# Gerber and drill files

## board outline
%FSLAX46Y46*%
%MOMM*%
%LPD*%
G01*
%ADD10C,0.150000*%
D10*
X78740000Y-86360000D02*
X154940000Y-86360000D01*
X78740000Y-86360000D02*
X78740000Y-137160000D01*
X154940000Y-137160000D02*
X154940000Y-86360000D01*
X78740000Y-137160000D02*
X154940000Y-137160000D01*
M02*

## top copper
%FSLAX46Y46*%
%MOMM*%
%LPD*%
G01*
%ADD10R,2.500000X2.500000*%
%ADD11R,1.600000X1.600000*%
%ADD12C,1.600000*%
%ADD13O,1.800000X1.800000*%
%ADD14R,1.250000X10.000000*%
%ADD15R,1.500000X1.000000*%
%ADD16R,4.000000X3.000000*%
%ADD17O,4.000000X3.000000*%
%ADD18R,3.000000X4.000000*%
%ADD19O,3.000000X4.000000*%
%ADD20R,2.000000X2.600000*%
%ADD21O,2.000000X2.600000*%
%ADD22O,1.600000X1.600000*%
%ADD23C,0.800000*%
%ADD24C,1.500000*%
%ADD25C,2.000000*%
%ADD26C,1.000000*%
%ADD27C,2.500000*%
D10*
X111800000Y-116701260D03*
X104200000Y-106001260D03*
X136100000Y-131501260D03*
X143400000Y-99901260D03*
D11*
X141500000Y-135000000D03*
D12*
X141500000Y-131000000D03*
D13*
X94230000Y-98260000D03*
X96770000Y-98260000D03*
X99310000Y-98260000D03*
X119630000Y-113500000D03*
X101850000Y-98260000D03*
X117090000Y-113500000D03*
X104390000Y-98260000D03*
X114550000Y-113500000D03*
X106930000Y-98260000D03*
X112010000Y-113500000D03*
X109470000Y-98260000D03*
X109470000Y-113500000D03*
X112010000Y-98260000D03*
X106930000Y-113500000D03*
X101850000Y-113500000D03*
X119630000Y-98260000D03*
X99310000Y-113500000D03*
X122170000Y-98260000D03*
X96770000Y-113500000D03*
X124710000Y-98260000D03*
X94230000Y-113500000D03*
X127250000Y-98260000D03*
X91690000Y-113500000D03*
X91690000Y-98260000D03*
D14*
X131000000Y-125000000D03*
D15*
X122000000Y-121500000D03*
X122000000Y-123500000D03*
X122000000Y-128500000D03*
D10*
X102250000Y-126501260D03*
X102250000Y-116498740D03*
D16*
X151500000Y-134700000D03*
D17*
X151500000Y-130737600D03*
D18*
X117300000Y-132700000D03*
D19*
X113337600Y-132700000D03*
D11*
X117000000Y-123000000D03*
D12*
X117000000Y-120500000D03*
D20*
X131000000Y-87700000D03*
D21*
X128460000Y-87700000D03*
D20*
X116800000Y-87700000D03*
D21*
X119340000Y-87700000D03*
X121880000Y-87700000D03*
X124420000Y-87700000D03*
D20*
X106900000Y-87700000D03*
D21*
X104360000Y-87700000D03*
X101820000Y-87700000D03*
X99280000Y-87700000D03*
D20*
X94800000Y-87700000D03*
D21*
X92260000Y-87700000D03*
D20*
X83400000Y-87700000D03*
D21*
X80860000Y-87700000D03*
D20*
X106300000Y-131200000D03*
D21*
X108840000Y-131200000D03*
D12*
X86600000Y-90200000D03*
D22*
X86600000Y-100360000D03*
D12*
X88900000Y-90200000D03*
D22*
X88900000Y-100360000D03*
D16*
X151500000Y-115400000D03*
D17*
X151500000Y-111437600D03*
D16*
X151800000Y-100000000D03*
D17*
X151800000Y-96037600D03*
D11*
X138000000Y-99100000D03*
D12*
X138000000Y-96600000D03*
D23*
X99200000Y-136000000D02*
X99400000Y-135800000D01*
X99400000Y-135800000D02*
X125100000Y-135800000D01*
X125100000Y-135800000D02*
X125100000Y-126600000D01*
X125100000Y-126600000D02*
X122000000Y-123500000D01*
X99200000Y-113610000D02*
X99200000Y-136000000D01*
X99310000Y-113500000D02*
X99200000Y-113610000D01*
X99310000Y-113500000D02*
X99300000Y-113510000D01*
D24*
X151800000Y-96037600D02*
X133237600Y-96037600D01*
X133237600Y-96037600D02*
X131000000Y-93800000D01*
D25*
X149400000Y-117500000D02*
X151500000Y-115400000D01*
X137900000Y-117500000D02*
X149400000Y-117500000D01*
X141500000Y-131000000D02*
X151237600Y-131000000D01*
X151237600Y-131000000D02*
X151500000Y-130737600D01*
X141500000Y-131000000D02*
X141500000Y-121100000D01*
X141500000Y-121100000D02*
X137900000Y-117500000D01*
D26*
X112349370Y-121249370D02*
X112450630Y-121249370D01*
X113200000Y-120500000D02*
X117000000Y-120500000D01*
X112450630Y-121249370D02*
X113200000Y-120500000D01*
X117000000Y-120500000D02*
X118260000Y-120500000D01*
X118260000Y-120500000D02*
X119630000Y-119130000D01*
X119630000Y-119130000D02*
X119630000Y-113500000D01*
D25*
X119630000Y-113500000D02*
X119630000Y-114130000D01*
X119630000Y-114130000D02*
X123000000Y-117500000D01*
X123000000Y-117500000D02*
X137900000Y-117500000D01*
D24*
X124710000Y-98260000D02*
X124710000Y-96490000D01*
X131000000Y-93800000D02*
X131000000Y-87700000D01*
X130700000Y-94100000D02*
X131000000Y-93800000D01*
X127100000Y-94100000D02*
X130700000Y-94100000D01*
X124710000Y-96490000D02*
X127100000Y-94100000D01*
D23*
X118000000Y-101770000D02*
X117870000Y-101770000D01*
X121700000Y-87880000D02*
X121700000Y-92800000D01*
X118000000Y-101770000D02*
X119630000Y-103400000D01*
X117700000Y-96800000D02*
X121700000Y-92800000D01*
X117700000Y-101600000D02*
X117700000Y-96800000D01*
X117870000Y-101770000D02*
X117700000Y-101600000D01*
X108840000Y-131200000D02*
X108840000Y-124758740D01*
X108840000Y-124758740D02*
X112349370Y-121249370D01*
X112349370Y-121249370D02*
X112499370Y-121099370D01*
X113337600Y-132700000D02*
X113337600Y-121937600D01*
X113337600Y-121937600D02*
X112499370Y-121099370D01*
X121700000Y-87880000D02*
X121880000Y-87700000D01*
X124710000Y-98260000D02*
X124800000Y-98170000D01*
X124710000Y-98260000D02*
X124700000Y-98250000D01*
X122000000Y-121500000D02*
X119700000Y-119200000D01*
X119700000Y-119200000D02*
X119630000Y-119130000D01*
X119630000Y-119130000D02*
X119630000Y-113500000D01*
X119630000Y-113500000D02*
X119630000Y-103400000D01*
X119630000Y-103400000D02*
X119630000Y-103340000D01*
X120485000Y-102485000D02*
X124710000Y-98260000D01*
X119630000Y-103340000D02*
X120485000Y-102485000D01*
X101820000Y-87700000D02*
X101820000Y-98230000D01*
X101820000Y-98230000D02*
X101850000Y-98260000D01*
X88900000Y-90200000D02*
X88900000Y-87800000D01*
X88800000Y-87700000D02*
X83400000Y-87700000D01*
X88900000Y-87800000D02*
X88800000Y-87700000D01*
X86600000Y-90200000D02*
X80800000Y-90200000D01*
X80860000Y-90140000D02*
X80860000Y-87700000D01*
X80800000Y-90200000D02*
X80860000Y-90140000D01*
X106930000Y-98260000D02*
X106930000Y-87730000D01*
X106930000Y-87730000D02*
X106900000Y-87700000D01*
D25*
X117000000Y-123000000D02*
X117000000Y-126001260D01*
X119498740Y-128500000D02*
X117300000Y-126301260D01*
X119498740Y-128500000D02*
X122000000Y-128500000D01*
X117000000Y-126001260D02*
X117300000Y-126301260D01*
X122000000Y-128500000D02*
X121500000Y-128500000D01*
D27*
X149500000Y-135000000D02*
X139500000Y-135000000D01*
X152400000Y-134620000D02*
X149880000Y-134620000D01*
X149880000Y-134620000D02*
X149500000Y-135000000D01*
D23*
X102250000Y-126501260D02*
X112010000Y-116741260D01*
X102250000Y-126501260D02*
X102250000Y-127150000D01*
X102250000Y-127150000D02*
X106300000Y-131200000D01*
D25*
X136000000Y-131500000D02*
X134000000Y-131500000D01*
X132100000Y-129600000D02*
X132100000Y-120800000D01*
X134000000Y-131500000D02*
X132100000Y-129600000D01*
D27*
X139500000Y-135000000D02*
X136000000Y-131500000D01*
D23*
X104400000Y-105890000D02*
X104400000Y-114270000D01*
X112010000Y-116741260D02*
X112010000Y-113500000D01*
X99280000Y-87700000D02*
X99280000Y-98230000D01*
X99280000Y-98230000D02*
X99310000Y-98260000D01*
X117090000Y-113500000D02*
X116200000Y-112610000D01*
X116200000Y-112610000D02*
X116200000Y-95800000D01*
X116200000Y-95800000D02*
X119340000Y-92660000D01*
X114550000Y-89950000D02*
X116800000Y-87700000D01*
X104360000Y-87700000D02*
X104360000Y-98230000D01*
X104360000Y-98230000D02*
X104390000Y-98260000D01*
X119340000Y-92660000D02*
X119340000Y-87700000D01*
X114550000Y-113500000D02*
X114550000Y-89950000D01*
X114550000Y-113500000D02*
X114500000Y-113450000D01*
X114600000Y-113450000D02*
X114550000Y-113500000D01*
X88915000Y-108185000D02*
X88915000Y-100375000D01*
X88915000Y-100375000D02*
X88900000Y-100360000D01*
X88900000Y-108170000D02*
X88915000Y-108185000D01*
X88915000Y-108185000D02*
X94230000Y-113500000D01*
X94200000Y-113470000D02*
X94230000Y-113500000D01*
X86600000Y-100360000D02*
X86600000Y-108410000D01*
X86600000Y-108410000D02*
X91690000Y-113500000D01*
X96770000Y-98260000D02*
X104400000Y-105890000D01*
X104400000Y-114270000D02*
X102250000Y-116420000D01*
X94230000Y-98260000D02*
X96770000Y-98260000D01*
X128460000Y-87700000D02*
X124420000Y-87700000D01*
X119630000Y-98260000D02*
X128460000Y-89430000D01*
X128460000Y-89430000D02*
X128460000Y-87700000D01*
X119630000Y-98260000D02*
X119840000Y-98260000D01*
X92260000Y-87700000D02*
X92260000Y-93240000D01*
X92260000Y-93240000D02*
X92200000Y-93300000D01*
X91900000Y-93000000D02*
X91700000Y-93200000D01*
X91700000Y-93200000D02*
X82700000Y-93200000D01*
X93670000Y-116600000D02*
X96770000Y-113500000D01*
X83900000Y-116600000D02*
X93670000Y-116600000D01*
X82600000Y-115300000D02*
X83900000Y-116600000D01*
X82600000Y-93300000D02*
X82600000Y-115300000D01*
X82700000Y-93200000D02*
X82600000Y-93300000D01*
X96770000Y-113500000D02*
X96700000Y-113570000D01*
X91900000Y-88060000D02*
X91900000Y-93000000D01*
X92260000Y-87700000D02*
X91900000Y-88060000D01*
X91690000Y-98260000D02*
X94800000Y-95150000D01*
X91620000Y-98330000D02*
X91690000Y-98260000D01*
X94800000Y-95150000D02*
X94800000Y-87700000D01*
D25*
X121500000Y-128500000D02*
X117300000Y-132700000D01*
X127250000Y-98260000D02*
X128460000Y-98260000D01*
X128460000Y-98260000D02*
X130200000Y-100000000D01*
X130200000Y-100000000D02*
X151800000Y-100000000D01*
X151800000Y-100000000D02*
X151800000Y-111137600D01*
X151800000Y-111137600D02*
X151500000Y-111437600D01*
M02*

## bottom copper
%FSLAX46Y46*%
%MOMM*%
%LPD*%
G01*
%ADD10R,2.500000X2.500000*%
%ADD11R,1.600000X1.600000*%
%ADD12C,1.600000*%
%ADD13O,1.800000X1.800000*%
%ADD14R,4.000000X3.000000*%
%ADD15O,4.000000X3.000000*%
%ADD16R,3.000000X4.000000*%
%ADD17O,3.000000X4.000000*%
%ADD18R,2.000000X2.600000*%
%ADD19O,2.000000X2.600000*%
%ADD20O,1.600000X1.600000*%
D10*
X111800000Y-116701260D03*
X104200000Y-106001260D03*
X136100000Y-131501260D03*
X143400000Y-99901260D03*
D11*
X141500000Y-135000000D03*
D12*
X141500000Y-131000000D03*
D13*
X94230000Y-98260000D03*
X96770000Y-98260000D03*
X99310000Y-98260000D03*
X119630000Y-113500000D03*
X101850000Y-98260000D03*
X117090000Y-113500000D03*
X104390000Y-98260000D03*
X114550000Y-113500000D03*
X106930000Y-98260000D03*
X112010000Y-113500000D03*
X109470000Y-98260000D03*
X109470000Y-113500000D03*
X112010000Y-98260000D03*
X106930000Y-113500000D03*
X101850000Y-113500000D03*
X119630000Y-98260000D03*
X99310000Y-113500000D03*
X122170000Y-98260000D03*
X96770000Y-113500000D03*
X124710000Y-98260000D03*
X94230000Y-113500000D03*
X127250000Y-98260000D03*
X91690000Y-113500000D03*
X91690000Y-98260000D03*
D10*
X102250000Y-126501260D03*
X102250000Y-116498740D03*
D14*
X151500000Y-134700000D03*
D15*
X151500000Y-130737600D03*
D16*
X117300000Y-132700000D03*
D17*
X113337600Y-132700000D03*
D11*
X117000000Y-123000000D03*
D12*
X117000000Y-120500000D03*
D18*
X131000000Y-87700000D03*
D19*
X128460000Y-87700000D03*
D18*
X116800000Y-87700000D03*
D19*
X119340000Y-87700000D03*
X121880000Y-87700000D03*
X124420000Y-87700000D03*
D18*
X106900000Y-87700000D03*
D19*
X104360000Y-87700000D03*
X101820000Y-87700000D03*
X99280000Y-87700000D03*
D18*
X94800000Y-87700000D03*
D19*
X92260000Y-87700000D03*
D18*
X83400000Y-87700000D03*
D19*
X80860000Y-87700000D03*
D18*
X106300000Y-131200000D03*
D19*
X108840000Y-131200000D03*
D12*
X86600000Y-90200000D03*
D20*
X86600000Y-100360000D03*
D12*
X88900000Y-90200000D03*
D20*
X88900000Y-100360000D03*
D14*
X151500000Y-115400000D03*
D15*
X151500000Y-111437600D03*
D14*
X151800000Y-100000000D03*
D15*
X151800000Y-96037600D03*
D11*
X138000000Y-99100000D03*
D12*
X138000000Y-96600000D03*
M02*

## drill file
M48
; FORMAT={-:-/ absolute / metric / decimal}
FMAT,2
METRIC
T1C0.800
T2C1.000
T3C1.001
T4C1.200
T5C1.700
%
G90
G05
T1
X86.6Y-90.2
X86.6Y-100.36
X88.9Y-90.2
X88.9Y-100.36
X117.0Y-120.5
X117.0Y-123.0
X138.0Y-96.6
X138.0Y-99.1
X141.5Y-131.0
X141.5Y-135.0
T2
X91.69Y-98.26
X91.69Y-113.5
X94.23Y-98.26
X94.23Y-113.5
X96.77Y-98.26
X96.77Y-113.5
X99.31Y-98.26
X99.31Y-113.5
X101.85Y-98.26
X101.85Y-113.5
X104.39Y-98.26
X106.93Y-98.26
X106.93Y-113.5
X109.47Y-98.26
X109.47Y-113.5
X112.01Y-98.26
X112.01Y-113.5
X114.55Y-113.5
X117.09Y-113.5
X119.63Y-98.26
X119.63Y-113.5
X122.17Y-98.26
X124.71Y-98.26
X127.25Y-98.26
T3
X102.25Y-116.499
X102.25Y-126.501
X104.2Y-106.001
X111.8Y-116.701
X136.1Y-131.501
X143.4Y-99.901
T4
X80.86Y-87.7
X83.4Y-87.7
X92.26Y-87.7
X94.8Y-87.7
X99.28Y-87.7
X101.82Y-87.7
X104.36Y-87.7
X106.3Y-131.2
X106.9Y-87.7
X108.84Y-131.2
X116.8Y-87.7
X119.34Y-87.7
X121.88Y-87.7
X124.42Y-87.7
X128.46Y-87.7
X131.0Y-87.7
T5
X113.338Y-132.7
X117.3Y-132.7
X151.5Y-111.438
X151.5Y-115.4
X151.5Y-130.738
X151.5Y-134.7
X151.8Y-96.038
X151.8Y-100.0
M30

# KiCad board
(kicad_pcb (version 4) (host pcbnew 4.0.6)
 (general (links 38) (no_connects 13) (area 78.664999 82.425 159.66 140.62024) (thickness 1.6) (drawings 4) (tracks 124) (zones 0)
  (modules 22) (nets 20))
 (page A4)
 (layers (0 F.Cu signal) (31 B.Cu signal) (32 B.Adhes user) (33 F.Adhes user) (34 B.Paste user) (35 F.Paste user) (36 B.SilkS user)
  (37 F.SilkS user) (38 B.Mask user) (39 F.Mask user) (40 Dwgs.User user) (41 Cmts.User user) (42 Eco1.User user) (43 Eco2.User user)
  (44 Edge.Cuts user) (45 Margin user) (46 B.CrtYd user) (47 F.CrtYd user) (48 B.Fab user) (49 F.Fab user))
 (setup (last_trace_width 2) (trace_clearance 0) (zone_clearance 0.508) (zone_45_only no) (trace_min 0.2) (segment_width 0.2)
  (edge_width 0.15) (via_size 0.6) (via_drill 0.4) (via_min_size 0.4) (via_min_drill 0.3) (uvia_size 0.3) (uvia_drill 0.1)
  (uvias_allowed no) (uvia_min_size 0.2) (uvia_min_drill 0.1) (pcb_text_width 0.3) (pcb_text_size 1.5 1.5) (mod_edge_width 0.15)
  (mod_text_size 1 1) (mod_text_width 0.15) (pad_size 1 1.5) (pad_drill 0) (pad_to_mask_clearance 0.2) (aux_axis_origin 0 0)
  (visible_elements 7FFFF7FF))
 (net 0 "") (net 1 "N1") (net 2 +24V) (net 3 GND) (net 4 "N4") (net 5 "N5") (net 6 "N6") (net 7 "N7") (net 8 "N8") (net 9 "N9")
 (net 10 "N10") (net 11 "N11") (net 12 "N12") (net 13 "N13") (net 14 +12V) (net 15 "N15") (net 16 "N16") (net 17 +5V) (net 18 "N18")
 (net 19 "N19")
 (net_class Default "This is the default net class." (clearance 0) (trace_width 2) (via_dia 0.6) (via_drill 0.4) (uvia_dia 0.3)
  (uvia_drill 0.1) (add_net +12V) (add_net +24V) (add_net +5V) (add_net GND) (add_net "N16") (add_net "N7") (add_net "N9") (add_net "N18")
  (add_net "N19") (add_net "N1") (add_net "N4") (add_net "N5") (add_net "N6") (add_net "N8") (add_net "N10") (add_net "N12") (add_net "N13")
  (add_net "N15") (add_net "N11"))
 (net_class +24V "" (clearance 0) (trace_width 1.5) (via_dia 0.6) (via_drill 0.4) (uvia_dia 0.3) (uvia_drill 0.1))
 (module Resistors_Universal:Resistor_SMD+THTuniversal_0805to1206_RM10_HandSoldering (layer F.Cu) (at 111.8 111.7 90)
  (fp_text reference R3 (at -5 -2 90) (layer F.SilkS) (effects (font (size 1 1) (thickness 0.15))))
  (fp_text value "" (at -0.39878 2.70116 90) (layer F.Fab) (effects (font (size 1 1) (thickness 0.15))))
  (pad 1 thru_hole rect (at -5.00126 0 270) (size 2.5 2.5) (drill 1.00076) (layers *.Cu *.Mask) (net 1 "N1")))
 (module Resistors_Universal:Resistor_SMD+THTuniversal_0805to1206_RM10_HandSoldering (layer F.Cu) (at 104.2 101 90)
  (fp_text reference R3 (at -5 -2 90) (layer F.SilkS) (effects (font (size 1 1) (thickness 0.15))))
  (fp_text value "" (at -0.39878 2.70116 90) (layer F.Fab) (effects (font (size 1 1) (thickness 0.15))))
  (pad 1 thru_hole rect (at -5.00126 0 270) (size 2.5 2.5) (drill 1.00076) (layers *.Cu *.Mask) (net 1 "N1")))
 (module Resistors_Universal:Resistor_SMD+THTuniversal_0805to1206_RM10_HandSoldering (layer F.Cu) (at 136.1 126.5 90)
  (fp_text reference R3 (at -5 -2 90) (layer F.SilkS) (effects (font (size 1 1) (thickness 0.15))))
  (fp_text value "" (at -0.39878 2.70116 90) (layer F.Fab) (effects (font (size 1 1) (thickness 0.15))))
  (pad 1 thru_hole rect (at -5.00126 0 270) (size 2.5 2.5) (drill 1.00076) (layers *.Cu *.Mask) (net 1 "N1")))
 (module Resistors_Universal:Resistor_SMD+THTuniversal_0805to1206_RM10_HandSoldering (layer F.Cu) (at 143.4 94.9 90)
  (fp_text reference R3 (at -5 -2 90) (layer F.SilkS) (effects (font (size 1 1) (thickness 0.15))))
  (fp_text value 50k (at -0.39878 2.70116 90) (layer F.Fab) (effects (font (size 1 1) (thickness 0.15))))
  (pad 1 thru_hole rect (at -5.00126 0 270) (size 2.5 2.5) (drill 1.00076) (layers *.Cu *.Mask) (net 1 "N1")))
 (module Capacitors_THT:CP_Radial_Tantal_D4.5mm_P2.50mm (layer B.Cu) (at 141.5 135 90)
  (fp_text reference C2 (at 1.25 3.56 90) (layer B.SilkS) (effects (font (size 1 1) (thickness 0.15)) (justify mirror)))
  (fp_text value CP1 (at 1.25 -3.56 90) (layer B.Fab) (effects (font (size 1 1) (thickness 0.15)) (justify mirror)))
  (pad 1 thru_hole rect (at 0 0 90) (size 1.6 1.6) (drill 0.8) (layers *.Cu *.Mask) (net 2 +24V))
  (pad 2 thru_hole circle (at 4 0 90) (size 1.6 1.6) (drill 0.8) (layers *.Cu *.Mask) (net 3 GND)))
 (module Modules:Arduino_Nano (layer B.Cu) (at 127.25 113.5 90)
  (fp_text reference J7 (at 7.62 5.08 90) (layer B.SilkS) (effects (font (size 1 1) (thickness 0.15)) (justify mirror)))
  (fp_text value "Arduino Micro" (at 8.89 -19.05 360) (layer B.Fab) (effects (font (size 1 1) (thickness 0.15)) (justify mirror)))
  (pad 3.3V thru_hole oval (at 15.24 -33.02 90) (size 1.8 1.8) (drill 1) (layers *.Cu *.Mask) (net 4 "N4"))
  (pad AREF thru_hole oval (at 15.24 -30.48 90) (size 1.8 1.8) (drill 1) (layers *.Cu *.Mask) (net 4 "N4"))
  (pad A0 thru_hole oval (at 15.24 -27.94 90) (size 1.8 1.8) (drill 1) (layers *.Cu *.Mask) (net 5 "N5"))
  (pad GND thru_hole oval (at 0 -7.62 90) (size 1.8 1.8) (drill 1) (layers *.Cu *.Mask) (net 3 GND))
  (pad A1 thru_hole oval (at 15.24 -25.4 90) (size 1.8 1.8) (drill 1) (layers *.Cu *.Mask) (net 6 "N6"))
  (pad SDA thru_hole oval (at 0 -10.16 90) (size 1.8 1.8) (drill 1) (layers *.Cu *.Mask) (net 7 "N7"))
  (pad A2 thru_hole oval (at 15.24 -22.86 90) (size 1.8 1.8) (drill 1) (layers *.Cu *.Mask) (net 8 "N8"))
  (pad SCL thru_hole oval (at 0 -12.7 90) (size 1.8 1.8) (drill 1) (layers *.Cu *.Mask) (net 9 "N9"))
  (pad A3 thru_hole oval (at 15.24 -20.32 90) (size 1.8 1.8) (drill 1) (layers *.Cu *.Mask) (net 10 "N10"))
  (pad D4 thru_hole oval (at 0 -15.24 90) (size 1.8 1.8) (drill 1) (layers *.Cu *.Mask) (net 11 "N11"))
  (pad A4 thru_hole oval (at 15.24 -17.78 90) (size 1.8 1.8) (drill 1) (layers *.Cu *.Mask) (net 1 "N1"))
  (pad D5 thru_hole oval (at 0 -17.78 90) (size 1.8 1.8) (drill 1) (layers *.Cu *.Mask))
  (pad A5 thru_hole oval (at 15.24 -15.24 90) (size 1.8 1.8) (drill 1) (layers *.Cu *.Mask) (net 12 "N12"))
  (pad D6 thru_hole oval (at 0 -20.32 90) (size 1.8 1.8) (drill 1) (layers *.Cu *.Mask))
  (pad D8 thru_hole oval (at 0 -25.4 90) (size 1.8 1.8) (drill 1) (layers *.Cu *.Mask))
  (pad 5v thru_hole oval (at 15.24 -7.62 90) (size 1.8 1.8) (drill 1) (layers *.Cu *.Mask))
  (pad D9 thru_hole oval (at 0 -27.94 90) (size 1.8 1.8) (drill 1) (layers *.Cu *.Mask))
  (pad RS thru_hole oval (at 15.24 -5.08 90) (size 1.8 1.8) (drill 1) (layers *.Cu *.Mask))
  (pad D10 thru_hole oval (at 0 -30.48 90) (size 1.8 1.8) (drill 1) (layers *.Cu *.Mask))
  (pad GND thru_hole oval (at 15.24 -2.54 90) (size 1.8 1.8) (drill 1) (layers *.Cu *.Mask) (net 3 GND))
  (pad D11 thru_hole oval (at 0 -33.02 90) (size 1.8 1.8) (drill 1) (layers *.Cu *.Mask) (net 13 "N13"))
  (pad Vin thru_hole oval (at 15.24 0 90) (size 1.8 1.8) (drill 1) (layers *.Cu *.Mask) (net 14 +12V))
  (pad D12 thru_hole oval (at 0 -35.56 90) (size 1.8 1.8) (drill 1) (layers *.Cu *.Mask) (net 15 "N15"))
  (pad D13 thru_hole oval (at 15.24 -35.56 90) (size 1.8 1.8) (drill 1) (layers *.Cu *.Mask)))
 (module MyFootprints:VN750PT (layer F.Cu) (at 128 125 270)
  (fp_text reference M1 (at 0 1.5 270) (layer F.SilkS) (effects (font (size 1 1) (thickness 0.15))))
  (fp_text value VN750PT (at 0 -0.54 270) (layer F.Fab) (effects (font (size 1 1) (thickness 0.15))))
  (pad Vcc smd rect (at 0 -3 270) (size 10 1.25) (layers F.Cu F.Paste F.Mask))
  (pad GND smd rect (at -3.5 6 270) (size 1 1.5) (layers F.Cu F.Paste F.Mask))
  (pad Inpu smd rect (at -1.5 6 270) (size 1 1.5) (layers F.Cu F.Paste F.Mask))
  (pad Vout smd rect (at 3.5 6 270) (size 1 1.5) (layers F.Cu F.Paste F.Mask) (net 2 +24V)))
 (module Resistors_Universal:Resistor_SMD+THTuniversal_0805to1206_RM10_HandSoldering (layer F.Cu) (at 102.25 121.5 90)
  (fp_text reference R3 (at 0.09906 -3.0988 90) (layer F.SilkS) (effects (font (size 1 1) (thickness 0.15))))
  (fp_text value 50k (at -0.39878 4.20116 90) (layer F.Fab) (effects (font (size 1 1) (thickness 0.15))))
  (pad 1 thru_hole rect (at -5.00126 0 270) (size 2.5 2.5) (drill 1.00076) (layers *.Cu *.Mask) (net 1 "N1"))
  (pad 2 thru_hole rect (at 5.00126 0 270) (size 2.5 2.5) (drill 1.00076) (layers *.Cu *.Mask) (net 4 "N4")))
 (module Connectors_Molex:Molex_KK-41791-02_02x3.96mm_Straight (layer F.Cu) (at 151.5 134.7 90)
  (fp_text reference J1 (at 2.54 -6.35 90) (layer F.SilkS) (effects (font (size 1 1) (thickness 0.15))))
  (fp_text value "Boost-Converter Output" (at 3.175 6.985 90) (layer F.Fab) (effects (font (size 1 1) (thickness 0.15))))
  (pad 1 thru_hole rect (at 0 0 90) (size 3 4) (drill 1.7) (layers *.Cu *.Mask) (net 2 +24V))
  (pad 2 thru_hole oval (at 3.9624 0 90) (size 3 4) (drill 1.7) (layers *.Cu *.Mask) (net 3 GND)))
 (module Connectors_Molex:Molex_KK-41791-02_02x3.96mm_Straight (layer B.Cu) (at 117.3 132.7 180)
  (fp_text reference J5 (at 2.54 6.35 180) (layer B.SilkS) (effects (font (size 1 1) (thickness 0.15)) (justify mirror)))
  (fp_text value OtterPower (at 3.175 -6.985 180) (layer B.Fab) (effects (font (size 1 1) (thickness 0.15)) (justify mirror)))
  (pad 1 thru_hole rect (at 0 0 180) (size 3 4) (drill 1.7) (layers *.Cu *.Mask) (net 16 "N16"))
  (pad 2 thru_hole oval (at 3.9624 0 180) (size 3 4) (drill 1.7) (layers *.Cu *.Mask) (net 3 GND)))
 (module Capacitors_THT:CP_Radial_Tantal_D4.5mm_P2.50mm (layer B.Cu) (at 117 123 90)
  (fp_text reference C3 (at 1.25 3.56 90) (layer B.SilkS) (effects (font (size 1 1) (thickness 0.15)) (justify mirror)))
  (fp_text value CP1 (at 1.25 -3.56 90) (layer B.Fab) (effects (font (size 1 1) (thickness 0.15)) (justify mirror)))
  (pad + thru_hole rect (at 0 0 90) (size 1.6 1.6) (drill 0.8) (layers *.Cu *.Mask) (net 2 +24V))
  (pad 2 thru_hole circle (at 2.5 0 90) (size 1.6 1.6) (drill 0.8) (layers *.Cu *.Mask) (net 3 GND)))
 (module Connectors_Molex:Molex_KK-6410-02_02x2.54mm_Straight (layer F.Cu) (at 131 87.7 180)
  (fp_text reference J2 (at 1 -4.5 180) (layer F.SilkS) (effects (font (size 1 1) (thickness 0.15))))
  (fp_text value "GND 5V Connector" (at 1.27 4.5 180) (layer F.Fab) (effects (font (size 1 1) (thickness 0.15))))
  (pad 1 thru_hole rect (at 0 0 180) (size 2 2.6) (drill 1.2) (layers *.Cu *.Mask) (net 3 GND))
  (pad 2 thru_hole oval (at 2.54 0 180) (size 2 2.6) (drill 1.2) (layers *.Cu *.Mask) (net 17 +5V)))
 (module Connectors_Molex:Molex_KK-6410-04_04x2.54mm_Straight (layer B.Cu) (at 116.8 87.7)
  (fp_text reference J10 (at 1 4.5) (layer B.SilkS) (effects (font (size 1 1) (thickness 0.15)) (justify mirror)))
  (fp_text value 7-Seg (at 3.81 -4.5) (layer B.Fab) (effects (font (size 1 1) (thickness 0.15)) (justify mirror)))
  (pad 1 thru_hole rect (at 0 0) (size 2 2.6) (drill 1.2) (layers *.Cu *.Mask) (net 7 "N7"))
  (pad 2 thru_hole oval (at 2.54 0) (size 2 2.6) (drill 1.2) (layers *.Cu *.Mask) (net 9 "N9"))
  (pad 3 thru_hole oval (at 5.08 0) (size 2 2.6) (drill 1.2) (layers *.Cu *.Mask) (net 3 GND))
  (pad 4 thru_hole oval (at 7.62 0) (size 2 2.6) (drill 1.2) (layers *.Cu *.Mask) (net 17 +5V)))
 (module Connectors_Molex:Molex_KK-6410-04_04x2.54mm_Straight (layer F.Cu) (at 106.9 87.7 180)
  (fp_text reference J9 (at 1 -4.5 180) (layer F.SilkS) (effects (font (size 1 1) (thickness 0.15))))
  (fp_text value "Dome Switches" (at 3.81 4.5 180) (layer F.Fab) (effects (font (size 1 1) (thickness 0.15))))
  (pad 1 thru_hole rect (at 0 0 180) (size 2 2.6) (drill 1.2) (layers *.Cu *.Mask) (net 10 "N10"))
  (pad 2 thru_hole oval (at 2.54 0 180) (size 2 2.6) (drill 1.2) (layers *.Cu *.Mask) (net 8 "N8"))
  (pad 3 thru_hole oval (at 5.08 0 180) (size 2 2.6) (drill 1.2) (layers *.Cu *.Mask) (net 6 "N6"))
  (pad 4 thru_hole oval (at 7.62 0 180) (size 2 2.6) (drill 1.2) (layers *.Cu *.Mask) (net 5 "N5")))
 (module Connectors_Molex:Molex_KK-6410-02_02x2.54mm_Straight (layer F.Cu) (at 94.8 87.7 180)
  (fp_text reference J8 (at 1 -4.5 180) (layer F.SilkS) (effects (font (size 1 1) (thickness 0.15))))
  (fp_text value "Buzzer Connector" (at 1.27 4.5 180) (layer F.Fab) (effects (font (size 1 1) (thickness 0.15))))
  (pad 1 thru_hole rect (at 0 0 180) (size 2 2.6) (drill 1.2) (layers *.Cu *.Mask) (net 12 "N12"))
  (pad 2 thru_hole oval (at 2.54 0 180) (size 2 2.6) (drill 1.2) (layers *.Cu *.Mask) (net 11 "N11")))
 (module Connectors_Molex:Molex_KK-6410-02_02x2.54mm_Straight (layer F.Cu) (at 83.4 87.7 180)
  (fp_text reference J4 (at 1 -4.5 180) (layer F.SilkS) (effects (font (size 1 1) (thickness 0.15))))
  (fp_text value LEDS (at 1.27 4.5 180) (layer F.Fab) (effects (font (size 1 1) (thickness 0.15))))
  (pad 1 thru_hole rect (at 0 0 180) (size 2 2.6) (drill 1.2) (layers *.Cu *.Mask) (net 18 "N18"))
  (pad 2 thru_hole oval (at 2.54 0 180) (size 2 2.6) (drill 1.2) (layers *.Cu *.Mask) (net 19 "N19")))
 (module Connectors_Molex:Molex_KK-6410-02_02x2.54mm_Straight (layer F.Cu) (at 106.3 131.2)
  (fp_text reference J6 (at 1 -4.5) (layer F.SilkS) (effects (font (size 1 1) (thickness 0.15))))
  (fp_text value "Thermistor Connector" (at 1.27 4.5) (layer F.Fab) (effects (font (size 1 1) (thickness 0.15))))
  (pad 1 thru_hole rect (at 0 0) (size 2 2.6) (drill 1.2) (layers *.Cu *.Mask) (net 1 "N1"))
  (pad 2 thru_hole oval (at 2.54 0) (size 2 2.6) (drill 1.2) (layers *.Cu *.Mask) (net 3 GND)))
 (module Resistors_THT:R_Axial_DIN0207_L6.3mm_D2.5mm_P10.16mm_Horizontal (layer F.Cu) (at 86.6 90.2 270)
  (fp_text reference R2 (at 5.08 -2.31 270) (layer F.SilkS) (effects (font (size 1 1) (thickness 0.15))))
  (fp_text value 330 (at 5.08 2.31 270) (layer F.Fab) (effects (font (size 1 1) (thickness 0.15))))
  (pad 1 thru_hole circle (at 0 0 270) (size 1.6 1.6) (drill 0.8) (layers *.Cu *.Mask) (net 19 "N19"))
  (pad 2 thru_hole oval (at 10.16 0 270) (size 1.6 1.6) (drill 0.8) (layers *.Cu *.Mask) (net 15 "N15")))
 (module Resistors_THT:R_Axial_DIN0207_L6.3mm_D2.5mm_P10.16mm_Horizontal (layer F.Cu) (at 88.9 90.2 270)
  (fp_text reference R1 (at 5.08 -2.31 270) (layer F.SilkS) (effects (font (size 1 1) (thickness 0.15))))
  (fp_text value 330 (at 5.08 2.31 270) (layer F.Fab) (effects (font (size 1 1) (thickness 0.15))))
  (pad 1 thru_hole circle (at 0 0 270) (size 1.6 1.6) (drill 0.8) (layers *.Cu *.Mask) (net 18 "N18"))
  (pad 2 thru_hole oval (at 10.16 0 270) (size 1.6 1.6) (drill 0.8) (layers *.Cu *.Mask) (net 13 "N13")))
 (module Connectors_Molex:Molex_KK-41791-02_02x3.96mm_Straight (layer F.Cu) (at 151.5 115.4 90)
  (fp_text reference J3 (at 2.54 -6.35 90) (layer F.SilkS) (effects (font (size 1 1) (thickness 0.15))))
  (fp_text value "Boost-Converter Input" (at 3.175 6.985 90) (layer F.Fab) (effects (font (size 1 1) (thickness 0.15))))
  (pad 1 thru_hole rect (at 0 0 90) (size 3 4) (drill 1.7) (layers *.Cu *.Mask) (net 3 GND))
  (pad 2 thru_hole oval (at 3.9624 0 90) (size 3 4) (drill 1.7) (layers *.Cu *.Mask) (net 14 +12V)))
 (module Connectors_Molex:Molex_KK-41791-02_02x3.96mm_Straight (layer F.Cu) (at 151.8 100 90)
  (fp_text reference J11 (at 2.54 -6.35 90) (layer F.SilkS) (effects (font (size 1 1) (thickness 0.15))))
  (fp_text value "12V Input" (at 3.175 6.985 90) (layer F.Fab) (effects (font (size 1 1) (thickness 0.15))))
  (pad 1 thru_hole rect (at 0 0 90) (size 3 4) (drill 1.7) (layers *.Cu *.Mask) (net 14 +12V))
  (pad 2 thru_hole oval (at 3.9624 0 90) (size 3 4) (drill 1.7) (layers *.Cu *.Mask) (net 3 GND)))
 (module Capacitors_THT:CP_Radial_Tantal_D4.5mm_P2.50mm (layer F.Cu) (at 138 99.1 90)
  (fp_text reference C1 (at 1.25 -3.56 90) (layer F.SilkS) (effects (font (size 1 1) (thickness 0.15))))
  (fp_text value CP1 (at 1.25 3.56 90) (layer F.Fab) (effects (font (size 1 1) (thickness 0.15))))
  (pad 1 thru_hole rect (at 0 0 90) (size 1.6 1.6) (drill 0.8) (layers *.Cu *.Mask) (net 16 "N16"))
  (pad 2 thru_hole circle (at 2.5 0 90) (size 1.6 1.6) (drill 0.8) (layers *.Cu *.Mask) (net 3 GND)))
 (gr_line (start 78.74 86.36) (end 154.94 86.36) (angle 90) (layer Edge.Cuts) (width 0.15))
 (gr_line (start 78.74 86.36) (end 78.74 137.16) (angle 90) (layer Edge.Cuts) (width 0.15))
 (gr_line (start 154.94 137.16) (end 154.94 86.36) (angle 90) (layer Edge.Cuts) (width 0.15))
 (gr_line (start 78.74 137.16) (end 154.94 137.16) (angle 90) (layer Edge.Cuts) (width 0.15))
 (segment (start 99.2 136) (end 99.4 135.8) (width 0.8) (layer F.Cu) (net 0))
 (segment (start 99.4 135.8) (end 125.1 135.8) (width 0.8) (layer F.Cu) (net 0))
 (segment (start 125.1 135.8) (end 125.1 126.6) (width 0.8) (layer F.Cu) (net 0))
 (segment (start 125.1 126.6) (end 122 123.5) (width 0.8) (layer F.Cu) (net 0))
 (segment (start 99.2 113.61) (end 99.2 136) (width 0.8) (layer F.Cu) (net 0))
 (segment (start 99.31 113.5) (end 99.2 113.61) (width 0.8) (layer F.Cu) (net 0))
 (segment (start 99.31 113.5) (end 99.3 113.51) (width 0.8) (layer F.Cu) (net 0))
 (segment (start 151.8 96.0376) (end 133.2376 96.0376) (width 1.5) (layer F.Cu) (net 3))
 (segment (start 133.2376 96.0376) (end 131 93.8) (width 1.5) (layer F.Cu) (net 3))
 (segment (start 149.4 117.5) (end 151.5 115.4) (width 2) (layer F.Cu) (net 3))
 (segment (start 137.9 117.5) (end 149.4 117.5) (width 2) (layer F.Cu) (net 3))
 (segment (start 141.5 131) (end 151.2376 131) (width 2) (layer F.Cu) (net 3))
 (segment (start 151.2376 131) (end 151.5 130.7376) (width 2) (layer F.Cu) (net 3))
 (segment (start 141.5 131) (end 141.5 121.1) (width 2) (layer F.Cu) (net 3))
 (segment (start 141.5 121.1) (end 137.9 117.5) (width 2) (layer F.Cu) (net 3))
 (segment (start 112.34937 121.24937) (end 112.45063 121.24937) (width 1) (layer F.Cu) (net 3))
 (segment (start 113.2 120.5) (end 117 120.5) (width 1) (layer F.Cu) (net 3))
 (segment (start 112.45063 121.24937) (end 113.2 120.5) (width 1) (layer F.Cu) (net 3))
 (segment (start 117 120.5) (end 118.26 120.5) (width 1) (layer F.Cu) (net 3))
 (segment (start 118.26 120.5) (end 119.63 119.13) (width 1) (layer F.Cu) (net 3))
 (segment (start 119.63 119.13) (end 119.63 113.5) (width 1) (layer F.Cu) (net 3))
 (segment (start 119.63 113.5) (end 119.63 114.13) (width 2) (layer F.Cu) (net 3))
 (segment (start 119.63 114.13) (end 123 117.5) (width 2) (layer F.Cu) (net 3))
 (segment (start 123 117.5) (end 137.9 117.5) (width 2) (layer F.Cu) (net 3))
 (segment (start 124.71 98.26) (end 124.71 96.49) (width 1.5) (layer F.Cu) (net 3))
 (segment (start 131 93.8) (end 131 87.7) (width 1.5) (layer F.Cu) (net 3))
 (segment (start 130.7 94.1) (end 131 93.8) (width 1.5) (layer F.Cu) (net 3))
 (segment (start 127.1 94.1) (end 130.7 94.1) (width 1.5) (layer F.Cu) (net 3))
 (segment (start 124.71 96.49) (end 127.1 94.1) (width 1.5) (layer F.Cu) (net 3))
 (segment (start 118 101.77) (end 117.87 101.77) (width 0.8) (layer F.Cu) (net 3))
 (segment (start 121.7 87.88) (end 121.7 92.8) (width 0.8) (layer F.Cu) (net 3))
 (segment (start 118 101.77) (end 119.63 103.4) (width 0.8) (layer F.Cu) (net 3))
 (segment (start 117.7 96.8) (end 121.7 92.8) (width 0.8) (layer F.Cu) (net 3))
 (segment (start 117.7 101.6) (end 117.7 96.8) (width 0.8) (layer F.Cu) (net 3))
 (segment (start 117.87 101.77) (end 117.7 101.6) (width 0.8) (layer F.Cu) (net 3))
 (segment (start 108.84 131.2) (end 108.84 124.75874) (width 0.8) (layer F.Cu) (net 3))
 (segment (start 108.84 124.75874) (end 112.34937 121.24937) (width 0.8) (layer F.Cu) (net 3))
 (segment (start 112.34937 121.24937) (end 112.49937 121.09937) (width 0.8) (layer F.Cu) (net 3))
 (segment (start 113.3376 132.7) (end 113.3376 121.9376) (width 0.8) (layer F.Cu) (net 3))
 (segment (start 113.3376 121.9376) (end 112.49937 121.09937) (width 0.8) (layer F.Cu) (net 3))
 (segment (start 121.7 87.88) (end 121.88 87.7) (width 0.8) (layer F.Cu) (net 3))
 (segment (start 124.71 98.26) (end 124.8 98.17) (width 0.8) (layer F.Cu) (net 3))
 (segment (start 124.71 98.26) (end 124.7 98.25) (width 0.8) (layer F.Cu) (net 3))
 (segment (start 122 121.5) (end 119.7 119.2) (width 0.8) (layer F.Cu) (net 3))
 (segment (start 119.7 119.2) (end 119.63 119.13) (width 0.8) (layer F.Cu) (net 3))
 (segment (start 119.63 119.13) (end 119.63 113.5) (width 0.8) (layer F.Cu) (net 3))
 (segment (start 119.63 113.5) (end 119.63 103.4) (width 0.8) (layer F.Cu) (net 3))
 (segment (start 119.63 103.4) (end 119.63 103.34) (width 0.8) (layer F.Cu) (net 3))
 (segment (start 120.485 102.485) (end 124.71 98.26) (width 0.8) (layer F.Cu) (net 3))
 (segment (start 119.63 103.34) (end 120.485 102.485) (width 0.8) (layer F.Cu) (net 3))
 (segment (start 101.82 87.7) (end 101.82 98.23) (width 0.8) (layer F.Cu) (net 6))
 (segment (start 101.82 98.23) (end 101.85 98.26) (width 0.8) (layer F.Cu) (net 6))
 (segment (start 88.9 90.2) (end 88.9 87.8) (width 0.8) (layer F.Cu) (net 18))
 (segment (start 88.8 87.7) (end 83.4 87.7) (width 0.8) (layer F.Cu) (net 18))
 (segment (start 88.9 87.8) (end 88.8 87.7) (width 0.8) (layer F.Cu) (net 18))
 (segment (start 86.6 90.2) (end 80.8 90.2) (width 0.8) (layer F.Cu) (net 19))
 (segment (start 80.86 90.14) (end 80.86 87.7) (width 0.8) (layer F.Cu) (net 19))
 (segment (start 80.8 90.2) (end 80.86 90.14) (width 0.8) (layer F.Cu) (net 19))
 (segment (start 106.93 98.26) (end 106.93 87.73) (width 0.8) (layer F.Cu) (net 10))
 (segment (start 106.93 87.73) (end 106.9 87.7) (width 0.8) (layer F.Cu) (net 10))
 (segment (start 117 123) (end 117 126.00126) (width 2) (layer F.Cu) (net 2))
 (segment (start 119.49874 128.5) (end 117.3 126.30126) (width 2) (layer F.Cu) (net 2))
 (segment (start 119.49874 128.5) (end 122 128.5) (width 2) (layer F.Cu) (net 2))
 (segment (start 117 126.00126) (end 117.3 126.30126) (width 2) (layer F.Cu) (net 2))
 (segment (start 122 128.5) (end 121.5 128.5) (width 2) (layer F.Cu) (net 2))
 (segment (start 149.5 135) (end 139.5 135) (width 2.5) (layer F.Cu) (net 2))
 (segment (start 152.4 134.62) (end 149.88 134.62) (width 2.5) (layer F.Cu) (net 2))
 (segment (start 149.88 134.62) (end 149.5 135) (width 2.5) (layer F.Cu) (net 2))
 (segment (start 102.25 126.50126) (end 112.01 116.74126) (width 0.8) (layer F.Cu) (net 1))
 (segment (start 102.25 126.50126) (end 102.25 127.15) (width 0.8) (layer F.Cu) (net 1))
 (segment (start 102.25 127.15) (end 106.3 131.2) (width 0.8) (layer F.Cu) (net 1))
 (segment (start 136 131.5) (end 134 131.5) (width 2) (layer F.Cu) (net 1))
 (segment (start 132.1 129.6) (end 132.1 120.8) (width 2) (layer F.Cu) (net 1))
 (segment (start 134 131.5) (end 132.1 129.6) (width 2) (layer F.Cu) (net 1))
 (segment (start 139.5 135) (end 136 131.5) (width 2.5) (layer F.Cu) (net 1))
 (segment (start 104.4 105.89) (end 104.4 114.27) (width 0.8) (layer F.Cu) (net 1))
 (segment (start 112.01 116.74126) (end 112.01 113.5) (width 0.8) (layer F.Cu) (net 1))
 (segment (start 99.28 87.7) (end 99.28 98.23) (width 0.8) (layer F.Cu) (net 5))
 (segment (start 99.28 98.23) (end 99.31 98.26) (width 0.8) (layer F.Cu) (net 5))
 (segment (start 117.09 113.5) (end 116.2 112.61) (width 0.8) (layer F.Cu) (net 7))
 (segment (start 116.2 112.61) (end 116.2 95.8) (width 0.8) (layer F.Cu) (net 7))
 (segment (start 116.2 95.8) (end 119.34 92.66) (width 0.8) (layer F.Cu) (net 7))
 (segment (start 114.55 89.95) (end 116.8 87.7) (width 0.8) (layer F.Cu) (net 7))
 (segment (start 104.36 87.7) (end 104.36 98.23) (width 0.8) (layer F.Cu) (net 8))
 (segment (start 104.36 98.23) (end 104.39 98.26) (width 0.8) (layer F.Cu) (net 8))
 (segment (start 119.34 92.66) (end 119.34 87.7) (width 0.8) (layer F.Cu) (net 9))
 (segment (start 114.55 113.5) (end 114.55 89.95) (width 0.8) (layer F.Cu) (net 9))
 (segment (start 114.55 113.5) (end 114.5 113.45) (width 0.8) (layer F.Cu) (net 9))
 (segment (start 114.6 113.45) (end 114.55 113.5) (width 0.8) (layer F.Cu) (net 9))
 (segment (start 88.915 108.185) (end 88.915 100.375) (width 0.8) (layer F.Cu) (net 13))
 (segment (start 88.915 100.375) (end 88.9 100.36) (width 0.8) (layer F.Cu) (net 13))
 (segment (start 88.9 108.17) (end 88.915 108.185) (width 0.8) (layer F.Cu) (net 13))
 (segment (start 88.915 108.185) (end 94.23 113.5) (width 0.8) (layer F.Cu) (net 13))
 (segment (start 94.2 113.47) (end 94.23 113.5) (width 0.8) (layer F.Cu) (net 13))
 (segment (start 86.6 100.36) (end 86.6 108.41) (width 0.8) (layer F.Cu) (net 15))
 (segment (start 86.6 108.41) (end 91.69 113.5) (width 0.8) (layer F.Cu) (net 15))
 (segment (start 96.77 98.26) (end 104.4 105.89) (width 0.8) (layer F.Cu) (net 4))
 (segment (start 104.4 114.27) (end 102.25 116.42) (width 0.8) (layer F.Cu) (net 4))
 (segment (start 94.23 98.26) (end 96.77 98.26) (width 0.8) (layer F.Cu) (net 4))
 (segment (start 128.46 87.7) (end 124.42 87.7) (width 0.8) (layer F.Cu) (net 17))
 (segment (start 119.63 98.26) (end 128.46 89.43) (width 0.8) (layer F.Cu) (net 17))
 (segment (start 128.46 89.43) (end 128.46 87.7) (width 0.8) (layer F.Cu) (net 17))
 (segment (start 119.63 98.26) (end 119.84 98.26) (width 0.8) (layer F.Cu) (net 17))
 (segment (start 92.26 87.7) (end 92.26 93.24) (width 0.8) (layer F.Cu) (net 11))
 (segment (start 92.26 93.24) (end 92.2 93.3) (width 0.8) (layer F.Cu) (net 11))
 (segment (start 91.9 93) (end 91.7 93.2) (width 0.8) (layer F.Cu) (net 11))
 (segment (start 91.7 93.2) (end 82.7 93.2) (width 0.8) (layer F.Cu) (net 11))
 (segment (start 93.67 116.6) (end 96.77 113.5) (width 0.8) (layer F.Cu) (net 11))
 (segment (start 83.9 116.6) (end 93.67 116.6) (width 0.8) (layer F.Cu) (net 11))
 (segment (start 82.6 115.3) (end 83.9 116.6) (width 0.8) (layer F.Cu) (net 11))
 (segment (start 82.6 93.3) (end 82.6 115.3) (width 0.8) (layer F.Cu) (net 11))
 (segment (start 82.7 93.2) (end 82.6 93.3) (width 0.8) (layer F.Cu) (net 11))
 (segment (start 96.77 113.5) (end 96.7 113.57) (width 0.8) (layer F.Cu) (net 11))
 (segment (start 91.9 88.06) (end 91.9 93) (width 0.8) (layer F.Cu) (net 11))
 (segment (start 92.26 87.7) (end 91.9 88.06) (width 0.8) (layer F.Cu) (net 11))
 (segment (start 91.69 98.26) (end 94.8 95.15) (width 0.8) (layer F.Cu) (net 12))
 (segment (start 91.62 98.33) (end 91.69 98.26) (width 0.8) (layer F.Cu) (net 12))
 (segment (start 94.8 95.15) (end 94.8 87.7) (width 0.8) (layer F.Cu) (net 12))
 (segment (start 121.5 128.5) (end 117.3 132.7) (width 2) (layer F.Cu) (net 16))
 (segment (start 127.25 98.26) (end 128.46 98.26) (width 2) (layer F.Cu) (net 14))
 (segment (start 128.46 98.26) (end 130.2 100) (width 2) (layer F.Cu) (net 14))
 (segment (start 130.2 100) (end 151.8 100) (width 2) (layer F.Cu) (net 14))
 (segment (start 151.8 100) (end 151.8 111.1376) (width 2) (layer F.Cu) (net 14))
 (segment (start 151.8 111.1376) (end 151.5 111.4376) (width 2) (layer F.Cu) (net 14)))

